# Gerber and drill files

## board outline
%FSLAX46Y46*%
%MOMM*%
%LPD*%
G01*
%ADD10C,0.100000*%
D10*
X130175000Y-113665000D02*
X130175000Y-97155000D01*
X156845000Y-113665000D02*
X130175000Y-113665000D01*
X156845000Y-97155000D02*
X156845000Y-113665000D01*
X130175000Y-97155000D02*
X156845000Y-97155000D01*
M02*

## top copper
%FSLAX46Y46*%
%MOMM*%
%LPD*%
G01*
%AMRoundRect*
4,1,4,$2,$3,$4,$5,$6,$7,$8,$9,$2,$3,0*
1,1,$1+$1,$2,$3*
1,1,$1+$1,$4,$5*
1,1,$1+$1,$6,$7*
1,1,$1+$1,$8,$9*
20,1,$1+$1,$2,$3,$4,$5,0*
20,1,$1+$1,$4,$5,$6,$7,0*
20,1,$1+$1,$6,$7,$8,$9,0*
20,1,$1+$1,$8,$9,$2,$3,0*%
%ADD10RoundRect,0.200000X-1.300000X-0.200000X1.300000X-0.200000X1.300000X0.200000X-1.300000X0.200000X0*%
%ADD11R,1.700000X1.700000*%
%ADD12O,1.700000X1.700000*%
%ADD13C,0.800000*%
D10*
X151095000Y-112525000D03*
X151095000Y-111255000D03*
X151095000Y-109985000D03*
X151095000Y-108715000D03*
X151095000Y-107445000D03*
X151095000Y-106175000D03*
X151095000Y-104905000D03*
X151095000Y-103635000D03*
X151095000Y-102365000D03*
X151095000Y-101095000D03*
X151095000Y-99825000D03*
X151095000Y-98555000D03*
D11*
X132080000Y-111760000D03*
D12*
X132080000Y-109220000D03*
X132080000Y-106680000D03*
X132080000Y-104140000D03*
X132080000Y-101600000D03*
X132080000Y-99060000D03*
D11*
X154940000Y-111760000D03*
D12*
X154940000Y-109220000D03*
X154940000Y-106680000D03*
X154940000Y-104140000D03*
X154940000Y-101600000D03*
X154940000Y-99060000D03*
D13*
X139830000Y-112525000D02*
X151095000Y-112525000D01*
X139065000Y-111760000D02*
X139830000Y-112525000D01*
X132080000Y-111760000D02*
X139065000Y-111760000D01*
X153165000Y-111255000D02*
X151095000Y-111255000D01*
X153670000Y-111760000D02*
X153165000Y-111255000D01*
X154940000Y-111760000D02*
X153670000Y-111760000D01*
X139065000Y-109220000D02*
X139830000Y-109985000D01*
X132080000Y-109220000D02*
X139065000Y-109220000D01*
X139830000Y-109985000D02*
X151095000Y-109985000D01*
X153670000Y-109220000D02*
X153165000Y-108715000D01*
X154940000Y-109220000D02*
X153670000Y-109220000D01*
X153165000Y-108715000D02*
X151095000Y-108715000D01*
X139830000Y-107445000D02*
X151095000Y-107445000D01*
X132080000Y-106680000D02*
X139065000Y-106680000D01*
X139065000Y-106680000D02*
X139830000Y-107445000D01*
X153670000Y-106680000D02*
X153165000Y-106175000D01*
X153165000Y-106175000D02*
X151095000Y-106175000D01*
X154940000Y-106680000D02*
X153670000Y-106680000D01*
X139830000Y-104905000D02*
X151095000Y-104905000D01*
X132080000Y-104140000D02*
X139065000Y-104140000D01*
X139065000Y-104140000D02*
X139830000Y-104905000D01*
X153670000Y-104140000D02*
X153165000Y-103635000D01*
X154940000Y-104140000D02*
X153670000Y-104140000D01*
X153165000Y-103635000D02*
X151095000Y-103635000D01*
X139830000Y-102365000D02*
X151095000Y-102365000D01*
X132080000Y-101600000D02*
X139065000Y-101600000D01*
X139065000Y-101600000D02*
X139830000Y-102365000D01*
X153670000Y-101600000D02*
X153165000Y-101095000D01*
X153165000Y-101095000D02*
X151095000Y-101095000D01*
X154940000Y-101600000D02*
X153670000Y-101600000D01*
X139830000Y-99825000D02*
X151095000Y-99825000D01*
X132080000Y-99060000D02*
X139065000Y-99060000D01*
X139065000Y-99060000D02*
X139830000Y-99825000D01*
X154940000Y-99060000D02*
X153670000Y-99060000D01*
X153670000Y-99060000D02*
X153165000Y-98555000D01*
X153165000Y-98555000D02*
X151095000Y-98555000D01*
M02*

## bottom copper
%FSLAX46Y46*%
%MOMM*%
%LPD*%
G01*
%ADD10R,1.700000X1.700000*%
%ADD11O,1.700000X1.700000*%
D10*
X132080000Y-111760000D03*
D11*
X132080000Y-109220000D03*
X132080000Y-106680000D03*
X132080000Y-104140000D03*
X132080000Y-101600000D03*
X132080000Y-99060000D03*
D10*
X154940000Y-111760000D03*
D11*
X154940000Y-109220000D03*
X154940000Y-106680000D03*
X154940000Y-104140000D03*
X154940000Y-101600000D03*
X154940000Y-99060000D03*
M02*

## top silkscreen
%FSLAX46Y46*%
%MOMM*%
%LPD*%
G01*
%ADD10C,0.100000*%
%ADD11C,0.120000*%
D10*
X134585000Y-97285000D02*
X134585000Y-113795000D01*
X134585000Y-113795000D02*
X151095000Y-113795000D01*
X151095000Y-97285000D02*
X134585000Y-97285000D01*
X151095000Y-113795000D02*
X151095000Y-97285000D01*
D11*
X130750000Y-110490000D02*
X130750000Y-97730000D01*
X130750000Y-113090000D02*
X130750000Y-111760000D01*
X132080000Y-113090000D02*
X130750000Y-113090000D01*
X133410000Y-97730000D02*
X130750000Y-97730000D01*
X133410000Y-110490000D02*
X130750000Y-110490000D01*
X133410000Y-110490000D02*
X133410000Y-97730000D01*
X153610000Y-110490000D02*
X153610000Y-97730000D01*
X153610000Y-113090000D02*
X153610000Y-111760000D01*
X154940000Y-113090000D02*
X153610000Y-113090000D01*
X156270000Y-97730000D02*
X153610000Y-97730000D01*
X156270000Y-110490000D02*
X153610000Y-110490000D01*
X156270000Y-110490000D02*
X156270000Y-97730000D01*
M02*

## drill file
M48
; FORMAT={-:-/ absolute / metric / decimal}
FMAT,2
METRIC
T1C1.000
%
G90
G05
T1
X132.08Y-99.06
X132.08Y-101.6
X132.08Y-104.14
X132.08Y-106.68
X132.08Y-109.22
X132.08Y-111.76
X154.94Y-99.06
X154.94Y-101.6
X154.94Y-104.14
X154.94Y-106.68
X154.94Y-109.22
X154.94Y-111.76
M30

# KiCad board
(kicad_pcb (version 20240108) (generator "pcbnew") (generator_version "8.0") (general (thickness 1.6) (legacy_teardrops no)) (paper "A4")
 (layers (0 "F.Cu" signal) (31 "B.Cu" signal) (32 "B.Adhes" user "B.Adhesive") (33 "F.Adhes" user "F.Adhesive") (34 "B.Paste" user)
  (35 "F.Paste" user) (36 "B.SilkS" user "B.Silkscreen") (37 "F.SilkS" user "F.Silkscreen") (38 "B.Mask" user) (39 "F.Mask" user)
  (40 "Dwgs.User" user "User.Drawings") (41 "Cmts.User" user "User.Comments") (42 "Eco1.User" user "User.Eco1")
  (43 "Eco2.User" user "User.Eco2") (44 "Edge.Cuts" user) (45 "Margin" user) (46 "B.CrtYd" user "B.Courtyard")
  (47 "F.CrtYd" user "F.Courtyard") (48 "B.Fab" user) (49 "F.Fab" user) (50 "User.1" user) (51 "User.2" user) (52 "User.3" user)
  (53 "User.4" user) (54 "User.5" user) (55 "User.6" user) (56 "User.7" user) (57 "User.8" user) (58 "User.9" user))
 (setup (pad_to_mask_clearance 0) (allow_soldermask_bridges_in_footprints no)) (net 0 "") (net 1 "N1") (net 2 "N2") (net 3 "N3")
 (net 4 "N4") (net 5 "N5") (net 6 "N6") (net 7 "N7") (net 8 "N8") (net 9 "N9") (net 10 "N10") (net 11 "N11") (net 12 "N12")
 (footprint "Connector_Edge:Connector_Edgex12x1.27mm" (layer "F.Cu") (at 151.095 115.065)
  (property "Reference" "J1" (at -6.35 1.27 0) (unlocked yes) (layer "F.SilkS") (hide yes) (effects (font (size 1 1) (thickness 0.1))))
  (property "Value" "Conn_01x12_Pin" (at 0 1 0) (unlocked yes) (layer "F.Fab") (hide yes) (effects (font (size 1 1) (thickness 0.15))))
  (fp_line (start -16.51 -17.78) (end -16.51 -1.27) (stroke (width 0.1) (type default)) (layer "F.SilkS"))
  (fp_line (start -16.51 -1.27) (end 0 -1.27) (stroke (width 0.1) (type default)) (layer "F.SilkS"))
  (fp_line (start 0 -17.78) (end -16.51 -17.78) (stroke (width 0.1) (type default)) (layer "F.SilkS"))
  (fp_line (start 0 -1.27) (end 0 -17.78) (stroke (width 0.1) (type default)) (layer "F.SilkS"))
  (pad "1" smd roundrect (at 0 -2.54) (size 3 0.8) (layers "F.Cu" "F.Paste" "F.Mask") (roundrect_rratio 0.25) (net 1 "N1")
   (thermal_bridge_angle 45))
  (pad "2" smd roundrect (at 0 -3.81) (size 3 0.8) (layers "F.Cu" "F.Paste" "F.Mask") (roundrect_rratio 0.25) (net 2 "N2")
   (thermal_bridge_angle 45))
  (pad "3" smd roundrect (at 0 -5.08) (size 3 0.8) (layers "F.Cu" "F.Paste" "F.Mask") (roundrect_rratio 0.25) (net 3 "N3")
   (thermal_bridge_angle 45))
  (pad "4" smd roundrect (at 0 -6.35) (size 3 0.8) (layers "F.Cu" "F.Paste" "F.Mask") (roundrect_rratio 0.25) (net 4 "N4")
   (thermal_bridge_angle 45))
  (pad "5" smd roundrect (at 0 -7.62) (size 3 0.8) (layers "F.Cu" "F.Paste" "F.Mask") (roundrect_rratio 0.25) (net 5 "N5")
   (thermal_bridge_angle 45))
  (pad "6" smd roundrect (at 0 -8.89) (size 3 0.8) (layers "F.Cu" "F.Paste" "F.Mask") (roundrect_rratio 0.25) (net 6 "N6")
   (thermal_bridge_angle 45))
  (pad "7" smd roundrect (at 0 -10.16) (size 3 0.8) (layers "F.Cu" "F.Paste" "F.Mask") (roundrect_rratio 0.25) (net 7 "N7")
   (thermal_bridge_angle 45))
  (pad "8" smd roundrect (at 0 -11.43) (size 3 0.8) (layers "F.Cu" "F.Paste" "F.Mask") (roundrect_rratio 0.25) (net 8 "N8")
   (thermal_bridge_angle 45))
  (pad "9" smd roundrect (at 0 -12.7) (size 3 0.8) (layers "F.Cu" "F.Paste" "F.Mask") (roundrect_rratio 0.25) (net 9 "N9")
   (thermal_bridge_angle 45))
  (pad "10" smd roundrect (at 0 -13.97) (size 3 0.8) (layers "F.Cu" "F.Paste" "F.Mask") (roundrect_rratio 0.25) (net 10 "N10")
   (thermal_bridge_angle 45))
  (pad "11" smd roundrect (at 0 -15.24) (size 3 0.8) (layers "F.Cu" "F.Paste" "F.Mask") (roundrect_rratio 0.25) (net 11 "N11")
   (thermal_bridge_angle 45))
  (pad "12" smd roundrect (at 0 -16.51) (size 3 0.8) (layers "F.Cu" "F.Paste" "F.Mask") (roundrect_rratio 0.25) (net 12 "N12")
   (thermal_bridge_angle 45)))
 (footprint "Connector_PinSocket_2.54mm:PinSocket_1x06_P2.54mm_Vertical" (layer "F.Cu") (at 132.08 111.76 180)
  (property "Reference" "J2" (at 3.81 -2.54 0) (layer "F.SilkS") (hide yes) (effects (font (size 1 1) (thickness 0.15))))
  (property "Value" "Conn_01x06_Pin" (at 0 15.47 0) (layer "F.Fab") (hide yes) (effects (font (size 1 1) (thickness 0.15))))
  (fp_line (start 1.33 1.27) (end 1.33 14.03) (stroke (width 0.12) (type solid)) (layer "F.SilkS"))
  (fp_line (start 1.33 -1.33) (end 1.33 0) (stroke (width 0.12) (type solid)) (layer "F.SilkS"))
  (fp_line (start 0 -1.33) (end 1.33 -1.33) (stroke (width 0.12) (type solid)) (layer "F.SilkS"))
  (fp_line (start -1.33 14.03) (end 1.33 14.03) (stroke (width 0.12) (type solid)) (layer "F.SilkS"))
  (fp_line (start -1.33 1.27) (end 1.33 1.27) (stroke (width 0.12) (type solid)) (layer "F.SilkS"))
  (fp_line (start -1.33 1.27) (end -1.33 14.03) (stroke (width 0.12) (type solid)) (layer "F.SilkS"))
  (pad "1" thru_hole rect (at 0 0 180) (size 1.7 1.7) (drill 1) (layers "*.Cu" "*.Mask") (remove_unused_layers no) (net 1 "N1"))
  (pad "2" thru_hole oval (at 0 2.54 180) (size 1.7 1.7) (drill 1) (layers "*.Cu" "*.Mask") (remove_unused_layers no) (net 3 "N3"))
  (pad "3" thru_hole oval (at 0 5.08 180) (size 1.7 1.7) (drill 1) (layers "*.Cu" "*.Mask") (remove_unused_layers no) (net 5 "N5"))
  (pad "4" thru_hole oval (at 0 7.62 180) (size 1.7 1.7) (drill 1) (layers "*.Cu" "*.Mask") (remove_unused_layers no) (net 7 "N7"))
  (pad "5" thru_hole oval (at 0 10.16 180) (size 1.7 1.7) (drill 1) (layers "*.Cu" "*.Mask") (remove_unused_layers no) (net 9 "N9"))
  (pad "6" thru_hole oval (at 0 12.7 180) (size 1.7 1.7) (drill 1) (layers "*.Cu" "*.Mask") (remove_unused_layers no) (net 11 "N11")))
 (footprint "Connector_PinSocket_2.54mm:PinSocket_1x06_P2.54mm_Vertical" (layer "F.Cu") (at 154.94 111.76 180)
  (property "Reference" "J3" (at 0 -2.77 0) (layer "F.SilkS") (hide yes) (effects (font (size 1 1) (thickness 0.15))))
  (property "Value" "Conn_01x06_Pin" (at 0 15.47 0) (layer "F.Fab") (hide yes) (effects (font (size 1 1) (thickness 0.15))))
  (fp_line (start 1.33 1.27) (end 1.33 14.03) (stroke (width 0.12) (type solid)) (layer "F.SilkS"))
  (fp_line (start 1.33 -1.33) (end 1.33 0) (stroke (width 0.12) (type solid)) (layer "F.SilkS"))
  (fp_line (start 0 -1.33) (end 1.33 -1.33) (stroke (width 0.12) (type solid)) (layer "F.SilkS"))
  (fp_line (start -1.33 14.03) (end 1.33 14.03) (stroke (width 0.12) (type solid)) (layer "F.SilkS"))
  (fp_line (start -1.33 1.27) (end 1.33 1.27) (stroke (width 0.12) (type solid)) (layer "F.SilkS"))
  (fp_line (start -1.33 1.27) (end -1.33 14.03) (stroke (width 0.12) (type solid)) (layer "F.SilkS"))
  (pad "1" thru_hole rect (at 0 0 180) (size 1.7 1.7) (drill 1) (layers "*.Cu" "*.Mask") (remove_unused_layers no) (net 2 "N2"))
  (pad "2" thru_hole oval (at 0 2.54 180) (size 1.7 1.7) (drill 1) (layers "*.Cu" "*.Mask") (remove_unused_layers no) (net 4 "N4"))
  (pad "3" thru_hole oval (at 0 5.08 180) (size 1.7 1.7) (drill 1) (layers "*.Cu" "*.Mask") (remove_unused_layers no) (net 6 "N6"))
  (pad "4" thru_hole oval (at 0 7.62 180) (size 1.7 1.7) (drill 1) (layers "*.Cu" "*.Mask") (remove_unused_layers no) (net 8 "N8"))
  (pad "5" thru_hole oval (at 0 10.16 180) (size 1.7 1.7) (drill 1) (layers "*.Cu" "*.Mask") (remove_unused_layers no) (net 10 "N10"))
  (pad "6" thru_hole oval (at 0 12.7 180) (size 1.7 1.7) (drill 1) (layers "*.Cu" "*.Mask") (remove_unused_layers no) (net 12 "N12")))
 (gr_line (start 130.175 113.665) (end 130.175 97.155) (stroke (width 0.1) (type default)) (layer "Edge.Cuts"))
 (gr_line (start 156.845 113.665) (end 130.175 113.665) (stroke (width 0.1) (type default)) (layer "Edge.Cuts"))
 (gr_line (start 156.845 97.155) (end 156.845 113.665) (stroke (width 0.1) (type default)) (layer "Edge.Cuts"))
 (gr_line (start 130.175 97.155) (end 156.845 97.155) (stroke (width 0.1) (type default)) (layer "Edge.Cuts"))
 (segment (start 139.83 112.525) (end 151.095 112.525) (width 0.8) (layer "F.Cu") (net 1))
 (segment (start 139.065 111.76) (end 139.83 112.525) (width 0.8) (layer "F.Cu") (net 1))
 (segment (start 132.08 111.76) (end 139.065 111.76) (width 0.8) (layer "F.Cu") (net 1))
 (segment (start 153.165 111.255) (end 151.095 111.255) (width 0.8) (layer "F.Cu") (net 2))
 (segment (start 153.67 111.76) (end 153.165 111.255) (width 0.8) (layer "F.Cu") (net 2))
 (segment (start 154.94 111.76) (end 153.67 111.76) (width 0.8) (layer "F.Cu") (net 2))
 (segment (start 139.065 109.22) (end 139.83 109.985) (width 0.8) (layer "F.Cu") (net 3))
 (segment (start 132.08 109.22) (end 139.065 109.22) (width 0.8) (layer "F.Cu") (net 3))
 (segment (start 139.83 109.985) (end 151.095 109.985) (width 0.8) (layer "F.Cu") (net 3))
 (segment (start 153.67 109.22) (end 153.165 108.715) (width 0.8) (layer "F.Cu") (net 4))
 (segment (start 154.94 109.22) (end 153.67 109.22) (width 0.8) (layer "F.Cu") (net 4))
 (segment (start 153.165 108.715) (end 151.095 108.715) (width 0.8) (layer "F.Cu") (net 4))
 (segment (start 139.83 107.445) (end 151.095 107.445) (width 0.8) (layer "F.Cu") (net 5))
 (segment (start 132.08 106.68) (end 139.065 106.68) (width 0.8) (layer "F.Cu") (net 5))
 (segment (start 139.065 106.68) (end 139.83 107.445) (width 0.8) (layer "F.Cu") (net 5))
 (segment (start 153.67 106.68) (end 153.165 106.175) (width 0.8) (layer "F.Cu") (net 6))
 (segment (start 153.165 106.175) (end 151.095 106.175) (width 0.8) (layer "F.Cu") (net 6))
 (segment (start 154.94 106.68) (end 153.67 106.68) (width 0.8) (layer "F.Cu") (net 6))
 (segment (start 139.83 104.905) (end 151.095 104.905) (width 0.8) (layer "F.Cu") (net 7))
 (segment (start 132.08 104.14) (end 139.065 104.14) (width 0.8) (layer "F.Cu") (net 7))
 (segment (start 139.065 104.14) (end 139.83 104.905) (width 0.8) (layer "F.Cu") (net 7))
 (segment (start 153.67 104.14) (end 153.165 103.635) (width 0.8) (layer "F.Cu") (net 8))
 (segment (start 154.94 104.14) (end 153.67 104.14) (width 0.8) (layer "F.Cu") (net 8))
 (segment (start 153.165 103.635) (end 151.095 103.635) (width 0.8) (layer "F.Cu") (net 8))
 (segment (start 139.83 102.365) (end 151.095 102.365) (width 0.8) (layer "F.Cu") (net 9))
 (segment (start 132.08 101.6) (end 139.065 101.6) (width 0.8) (layer "F.Cu") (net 9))
 (segment (start 139.065 101.6) (end 139.83 102.365) (width 0.8) (layer "F.Cu") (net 9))
 (segment (start 153.67 101.6) (end 153.165 101.095) (width 0.8) (layer "F.Cu") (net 10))
 (segment (start 153.165 101.095) (end 151.095 101.095) (width 0.8) (layer "F.Cu") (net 10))
 (segment (start 154.94 101.6) (end 153.67 101.6) (width 0.8) (layer "F.Cu") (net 10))
 (segment (start 139.83 99.825) (end 151.095 99.825) (width 0.8) (layer "F.Cu") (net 11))
 (segment (start 132.08 99.06) (end 139.065 99.06) (width 0.8) (layer "F.Cu") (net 11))
 (segment (start 139.065 99.06) (end 139.83 99.825) (width 0.8) (layer "F.Cu") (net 11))
 (segment (start 154.94 99.06) (end 153.67 99.06) (width 0.8) (layer "F.Cu") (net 12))
 (segment (start 153.67 99.06) (end 153.165 98.555) (width 0.8) (layer "F.Cu") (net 12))
 (segment (start 153.165 98.555) (end 151.095 98.555) (width 0.8) (layer "F.Cu") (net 12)))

